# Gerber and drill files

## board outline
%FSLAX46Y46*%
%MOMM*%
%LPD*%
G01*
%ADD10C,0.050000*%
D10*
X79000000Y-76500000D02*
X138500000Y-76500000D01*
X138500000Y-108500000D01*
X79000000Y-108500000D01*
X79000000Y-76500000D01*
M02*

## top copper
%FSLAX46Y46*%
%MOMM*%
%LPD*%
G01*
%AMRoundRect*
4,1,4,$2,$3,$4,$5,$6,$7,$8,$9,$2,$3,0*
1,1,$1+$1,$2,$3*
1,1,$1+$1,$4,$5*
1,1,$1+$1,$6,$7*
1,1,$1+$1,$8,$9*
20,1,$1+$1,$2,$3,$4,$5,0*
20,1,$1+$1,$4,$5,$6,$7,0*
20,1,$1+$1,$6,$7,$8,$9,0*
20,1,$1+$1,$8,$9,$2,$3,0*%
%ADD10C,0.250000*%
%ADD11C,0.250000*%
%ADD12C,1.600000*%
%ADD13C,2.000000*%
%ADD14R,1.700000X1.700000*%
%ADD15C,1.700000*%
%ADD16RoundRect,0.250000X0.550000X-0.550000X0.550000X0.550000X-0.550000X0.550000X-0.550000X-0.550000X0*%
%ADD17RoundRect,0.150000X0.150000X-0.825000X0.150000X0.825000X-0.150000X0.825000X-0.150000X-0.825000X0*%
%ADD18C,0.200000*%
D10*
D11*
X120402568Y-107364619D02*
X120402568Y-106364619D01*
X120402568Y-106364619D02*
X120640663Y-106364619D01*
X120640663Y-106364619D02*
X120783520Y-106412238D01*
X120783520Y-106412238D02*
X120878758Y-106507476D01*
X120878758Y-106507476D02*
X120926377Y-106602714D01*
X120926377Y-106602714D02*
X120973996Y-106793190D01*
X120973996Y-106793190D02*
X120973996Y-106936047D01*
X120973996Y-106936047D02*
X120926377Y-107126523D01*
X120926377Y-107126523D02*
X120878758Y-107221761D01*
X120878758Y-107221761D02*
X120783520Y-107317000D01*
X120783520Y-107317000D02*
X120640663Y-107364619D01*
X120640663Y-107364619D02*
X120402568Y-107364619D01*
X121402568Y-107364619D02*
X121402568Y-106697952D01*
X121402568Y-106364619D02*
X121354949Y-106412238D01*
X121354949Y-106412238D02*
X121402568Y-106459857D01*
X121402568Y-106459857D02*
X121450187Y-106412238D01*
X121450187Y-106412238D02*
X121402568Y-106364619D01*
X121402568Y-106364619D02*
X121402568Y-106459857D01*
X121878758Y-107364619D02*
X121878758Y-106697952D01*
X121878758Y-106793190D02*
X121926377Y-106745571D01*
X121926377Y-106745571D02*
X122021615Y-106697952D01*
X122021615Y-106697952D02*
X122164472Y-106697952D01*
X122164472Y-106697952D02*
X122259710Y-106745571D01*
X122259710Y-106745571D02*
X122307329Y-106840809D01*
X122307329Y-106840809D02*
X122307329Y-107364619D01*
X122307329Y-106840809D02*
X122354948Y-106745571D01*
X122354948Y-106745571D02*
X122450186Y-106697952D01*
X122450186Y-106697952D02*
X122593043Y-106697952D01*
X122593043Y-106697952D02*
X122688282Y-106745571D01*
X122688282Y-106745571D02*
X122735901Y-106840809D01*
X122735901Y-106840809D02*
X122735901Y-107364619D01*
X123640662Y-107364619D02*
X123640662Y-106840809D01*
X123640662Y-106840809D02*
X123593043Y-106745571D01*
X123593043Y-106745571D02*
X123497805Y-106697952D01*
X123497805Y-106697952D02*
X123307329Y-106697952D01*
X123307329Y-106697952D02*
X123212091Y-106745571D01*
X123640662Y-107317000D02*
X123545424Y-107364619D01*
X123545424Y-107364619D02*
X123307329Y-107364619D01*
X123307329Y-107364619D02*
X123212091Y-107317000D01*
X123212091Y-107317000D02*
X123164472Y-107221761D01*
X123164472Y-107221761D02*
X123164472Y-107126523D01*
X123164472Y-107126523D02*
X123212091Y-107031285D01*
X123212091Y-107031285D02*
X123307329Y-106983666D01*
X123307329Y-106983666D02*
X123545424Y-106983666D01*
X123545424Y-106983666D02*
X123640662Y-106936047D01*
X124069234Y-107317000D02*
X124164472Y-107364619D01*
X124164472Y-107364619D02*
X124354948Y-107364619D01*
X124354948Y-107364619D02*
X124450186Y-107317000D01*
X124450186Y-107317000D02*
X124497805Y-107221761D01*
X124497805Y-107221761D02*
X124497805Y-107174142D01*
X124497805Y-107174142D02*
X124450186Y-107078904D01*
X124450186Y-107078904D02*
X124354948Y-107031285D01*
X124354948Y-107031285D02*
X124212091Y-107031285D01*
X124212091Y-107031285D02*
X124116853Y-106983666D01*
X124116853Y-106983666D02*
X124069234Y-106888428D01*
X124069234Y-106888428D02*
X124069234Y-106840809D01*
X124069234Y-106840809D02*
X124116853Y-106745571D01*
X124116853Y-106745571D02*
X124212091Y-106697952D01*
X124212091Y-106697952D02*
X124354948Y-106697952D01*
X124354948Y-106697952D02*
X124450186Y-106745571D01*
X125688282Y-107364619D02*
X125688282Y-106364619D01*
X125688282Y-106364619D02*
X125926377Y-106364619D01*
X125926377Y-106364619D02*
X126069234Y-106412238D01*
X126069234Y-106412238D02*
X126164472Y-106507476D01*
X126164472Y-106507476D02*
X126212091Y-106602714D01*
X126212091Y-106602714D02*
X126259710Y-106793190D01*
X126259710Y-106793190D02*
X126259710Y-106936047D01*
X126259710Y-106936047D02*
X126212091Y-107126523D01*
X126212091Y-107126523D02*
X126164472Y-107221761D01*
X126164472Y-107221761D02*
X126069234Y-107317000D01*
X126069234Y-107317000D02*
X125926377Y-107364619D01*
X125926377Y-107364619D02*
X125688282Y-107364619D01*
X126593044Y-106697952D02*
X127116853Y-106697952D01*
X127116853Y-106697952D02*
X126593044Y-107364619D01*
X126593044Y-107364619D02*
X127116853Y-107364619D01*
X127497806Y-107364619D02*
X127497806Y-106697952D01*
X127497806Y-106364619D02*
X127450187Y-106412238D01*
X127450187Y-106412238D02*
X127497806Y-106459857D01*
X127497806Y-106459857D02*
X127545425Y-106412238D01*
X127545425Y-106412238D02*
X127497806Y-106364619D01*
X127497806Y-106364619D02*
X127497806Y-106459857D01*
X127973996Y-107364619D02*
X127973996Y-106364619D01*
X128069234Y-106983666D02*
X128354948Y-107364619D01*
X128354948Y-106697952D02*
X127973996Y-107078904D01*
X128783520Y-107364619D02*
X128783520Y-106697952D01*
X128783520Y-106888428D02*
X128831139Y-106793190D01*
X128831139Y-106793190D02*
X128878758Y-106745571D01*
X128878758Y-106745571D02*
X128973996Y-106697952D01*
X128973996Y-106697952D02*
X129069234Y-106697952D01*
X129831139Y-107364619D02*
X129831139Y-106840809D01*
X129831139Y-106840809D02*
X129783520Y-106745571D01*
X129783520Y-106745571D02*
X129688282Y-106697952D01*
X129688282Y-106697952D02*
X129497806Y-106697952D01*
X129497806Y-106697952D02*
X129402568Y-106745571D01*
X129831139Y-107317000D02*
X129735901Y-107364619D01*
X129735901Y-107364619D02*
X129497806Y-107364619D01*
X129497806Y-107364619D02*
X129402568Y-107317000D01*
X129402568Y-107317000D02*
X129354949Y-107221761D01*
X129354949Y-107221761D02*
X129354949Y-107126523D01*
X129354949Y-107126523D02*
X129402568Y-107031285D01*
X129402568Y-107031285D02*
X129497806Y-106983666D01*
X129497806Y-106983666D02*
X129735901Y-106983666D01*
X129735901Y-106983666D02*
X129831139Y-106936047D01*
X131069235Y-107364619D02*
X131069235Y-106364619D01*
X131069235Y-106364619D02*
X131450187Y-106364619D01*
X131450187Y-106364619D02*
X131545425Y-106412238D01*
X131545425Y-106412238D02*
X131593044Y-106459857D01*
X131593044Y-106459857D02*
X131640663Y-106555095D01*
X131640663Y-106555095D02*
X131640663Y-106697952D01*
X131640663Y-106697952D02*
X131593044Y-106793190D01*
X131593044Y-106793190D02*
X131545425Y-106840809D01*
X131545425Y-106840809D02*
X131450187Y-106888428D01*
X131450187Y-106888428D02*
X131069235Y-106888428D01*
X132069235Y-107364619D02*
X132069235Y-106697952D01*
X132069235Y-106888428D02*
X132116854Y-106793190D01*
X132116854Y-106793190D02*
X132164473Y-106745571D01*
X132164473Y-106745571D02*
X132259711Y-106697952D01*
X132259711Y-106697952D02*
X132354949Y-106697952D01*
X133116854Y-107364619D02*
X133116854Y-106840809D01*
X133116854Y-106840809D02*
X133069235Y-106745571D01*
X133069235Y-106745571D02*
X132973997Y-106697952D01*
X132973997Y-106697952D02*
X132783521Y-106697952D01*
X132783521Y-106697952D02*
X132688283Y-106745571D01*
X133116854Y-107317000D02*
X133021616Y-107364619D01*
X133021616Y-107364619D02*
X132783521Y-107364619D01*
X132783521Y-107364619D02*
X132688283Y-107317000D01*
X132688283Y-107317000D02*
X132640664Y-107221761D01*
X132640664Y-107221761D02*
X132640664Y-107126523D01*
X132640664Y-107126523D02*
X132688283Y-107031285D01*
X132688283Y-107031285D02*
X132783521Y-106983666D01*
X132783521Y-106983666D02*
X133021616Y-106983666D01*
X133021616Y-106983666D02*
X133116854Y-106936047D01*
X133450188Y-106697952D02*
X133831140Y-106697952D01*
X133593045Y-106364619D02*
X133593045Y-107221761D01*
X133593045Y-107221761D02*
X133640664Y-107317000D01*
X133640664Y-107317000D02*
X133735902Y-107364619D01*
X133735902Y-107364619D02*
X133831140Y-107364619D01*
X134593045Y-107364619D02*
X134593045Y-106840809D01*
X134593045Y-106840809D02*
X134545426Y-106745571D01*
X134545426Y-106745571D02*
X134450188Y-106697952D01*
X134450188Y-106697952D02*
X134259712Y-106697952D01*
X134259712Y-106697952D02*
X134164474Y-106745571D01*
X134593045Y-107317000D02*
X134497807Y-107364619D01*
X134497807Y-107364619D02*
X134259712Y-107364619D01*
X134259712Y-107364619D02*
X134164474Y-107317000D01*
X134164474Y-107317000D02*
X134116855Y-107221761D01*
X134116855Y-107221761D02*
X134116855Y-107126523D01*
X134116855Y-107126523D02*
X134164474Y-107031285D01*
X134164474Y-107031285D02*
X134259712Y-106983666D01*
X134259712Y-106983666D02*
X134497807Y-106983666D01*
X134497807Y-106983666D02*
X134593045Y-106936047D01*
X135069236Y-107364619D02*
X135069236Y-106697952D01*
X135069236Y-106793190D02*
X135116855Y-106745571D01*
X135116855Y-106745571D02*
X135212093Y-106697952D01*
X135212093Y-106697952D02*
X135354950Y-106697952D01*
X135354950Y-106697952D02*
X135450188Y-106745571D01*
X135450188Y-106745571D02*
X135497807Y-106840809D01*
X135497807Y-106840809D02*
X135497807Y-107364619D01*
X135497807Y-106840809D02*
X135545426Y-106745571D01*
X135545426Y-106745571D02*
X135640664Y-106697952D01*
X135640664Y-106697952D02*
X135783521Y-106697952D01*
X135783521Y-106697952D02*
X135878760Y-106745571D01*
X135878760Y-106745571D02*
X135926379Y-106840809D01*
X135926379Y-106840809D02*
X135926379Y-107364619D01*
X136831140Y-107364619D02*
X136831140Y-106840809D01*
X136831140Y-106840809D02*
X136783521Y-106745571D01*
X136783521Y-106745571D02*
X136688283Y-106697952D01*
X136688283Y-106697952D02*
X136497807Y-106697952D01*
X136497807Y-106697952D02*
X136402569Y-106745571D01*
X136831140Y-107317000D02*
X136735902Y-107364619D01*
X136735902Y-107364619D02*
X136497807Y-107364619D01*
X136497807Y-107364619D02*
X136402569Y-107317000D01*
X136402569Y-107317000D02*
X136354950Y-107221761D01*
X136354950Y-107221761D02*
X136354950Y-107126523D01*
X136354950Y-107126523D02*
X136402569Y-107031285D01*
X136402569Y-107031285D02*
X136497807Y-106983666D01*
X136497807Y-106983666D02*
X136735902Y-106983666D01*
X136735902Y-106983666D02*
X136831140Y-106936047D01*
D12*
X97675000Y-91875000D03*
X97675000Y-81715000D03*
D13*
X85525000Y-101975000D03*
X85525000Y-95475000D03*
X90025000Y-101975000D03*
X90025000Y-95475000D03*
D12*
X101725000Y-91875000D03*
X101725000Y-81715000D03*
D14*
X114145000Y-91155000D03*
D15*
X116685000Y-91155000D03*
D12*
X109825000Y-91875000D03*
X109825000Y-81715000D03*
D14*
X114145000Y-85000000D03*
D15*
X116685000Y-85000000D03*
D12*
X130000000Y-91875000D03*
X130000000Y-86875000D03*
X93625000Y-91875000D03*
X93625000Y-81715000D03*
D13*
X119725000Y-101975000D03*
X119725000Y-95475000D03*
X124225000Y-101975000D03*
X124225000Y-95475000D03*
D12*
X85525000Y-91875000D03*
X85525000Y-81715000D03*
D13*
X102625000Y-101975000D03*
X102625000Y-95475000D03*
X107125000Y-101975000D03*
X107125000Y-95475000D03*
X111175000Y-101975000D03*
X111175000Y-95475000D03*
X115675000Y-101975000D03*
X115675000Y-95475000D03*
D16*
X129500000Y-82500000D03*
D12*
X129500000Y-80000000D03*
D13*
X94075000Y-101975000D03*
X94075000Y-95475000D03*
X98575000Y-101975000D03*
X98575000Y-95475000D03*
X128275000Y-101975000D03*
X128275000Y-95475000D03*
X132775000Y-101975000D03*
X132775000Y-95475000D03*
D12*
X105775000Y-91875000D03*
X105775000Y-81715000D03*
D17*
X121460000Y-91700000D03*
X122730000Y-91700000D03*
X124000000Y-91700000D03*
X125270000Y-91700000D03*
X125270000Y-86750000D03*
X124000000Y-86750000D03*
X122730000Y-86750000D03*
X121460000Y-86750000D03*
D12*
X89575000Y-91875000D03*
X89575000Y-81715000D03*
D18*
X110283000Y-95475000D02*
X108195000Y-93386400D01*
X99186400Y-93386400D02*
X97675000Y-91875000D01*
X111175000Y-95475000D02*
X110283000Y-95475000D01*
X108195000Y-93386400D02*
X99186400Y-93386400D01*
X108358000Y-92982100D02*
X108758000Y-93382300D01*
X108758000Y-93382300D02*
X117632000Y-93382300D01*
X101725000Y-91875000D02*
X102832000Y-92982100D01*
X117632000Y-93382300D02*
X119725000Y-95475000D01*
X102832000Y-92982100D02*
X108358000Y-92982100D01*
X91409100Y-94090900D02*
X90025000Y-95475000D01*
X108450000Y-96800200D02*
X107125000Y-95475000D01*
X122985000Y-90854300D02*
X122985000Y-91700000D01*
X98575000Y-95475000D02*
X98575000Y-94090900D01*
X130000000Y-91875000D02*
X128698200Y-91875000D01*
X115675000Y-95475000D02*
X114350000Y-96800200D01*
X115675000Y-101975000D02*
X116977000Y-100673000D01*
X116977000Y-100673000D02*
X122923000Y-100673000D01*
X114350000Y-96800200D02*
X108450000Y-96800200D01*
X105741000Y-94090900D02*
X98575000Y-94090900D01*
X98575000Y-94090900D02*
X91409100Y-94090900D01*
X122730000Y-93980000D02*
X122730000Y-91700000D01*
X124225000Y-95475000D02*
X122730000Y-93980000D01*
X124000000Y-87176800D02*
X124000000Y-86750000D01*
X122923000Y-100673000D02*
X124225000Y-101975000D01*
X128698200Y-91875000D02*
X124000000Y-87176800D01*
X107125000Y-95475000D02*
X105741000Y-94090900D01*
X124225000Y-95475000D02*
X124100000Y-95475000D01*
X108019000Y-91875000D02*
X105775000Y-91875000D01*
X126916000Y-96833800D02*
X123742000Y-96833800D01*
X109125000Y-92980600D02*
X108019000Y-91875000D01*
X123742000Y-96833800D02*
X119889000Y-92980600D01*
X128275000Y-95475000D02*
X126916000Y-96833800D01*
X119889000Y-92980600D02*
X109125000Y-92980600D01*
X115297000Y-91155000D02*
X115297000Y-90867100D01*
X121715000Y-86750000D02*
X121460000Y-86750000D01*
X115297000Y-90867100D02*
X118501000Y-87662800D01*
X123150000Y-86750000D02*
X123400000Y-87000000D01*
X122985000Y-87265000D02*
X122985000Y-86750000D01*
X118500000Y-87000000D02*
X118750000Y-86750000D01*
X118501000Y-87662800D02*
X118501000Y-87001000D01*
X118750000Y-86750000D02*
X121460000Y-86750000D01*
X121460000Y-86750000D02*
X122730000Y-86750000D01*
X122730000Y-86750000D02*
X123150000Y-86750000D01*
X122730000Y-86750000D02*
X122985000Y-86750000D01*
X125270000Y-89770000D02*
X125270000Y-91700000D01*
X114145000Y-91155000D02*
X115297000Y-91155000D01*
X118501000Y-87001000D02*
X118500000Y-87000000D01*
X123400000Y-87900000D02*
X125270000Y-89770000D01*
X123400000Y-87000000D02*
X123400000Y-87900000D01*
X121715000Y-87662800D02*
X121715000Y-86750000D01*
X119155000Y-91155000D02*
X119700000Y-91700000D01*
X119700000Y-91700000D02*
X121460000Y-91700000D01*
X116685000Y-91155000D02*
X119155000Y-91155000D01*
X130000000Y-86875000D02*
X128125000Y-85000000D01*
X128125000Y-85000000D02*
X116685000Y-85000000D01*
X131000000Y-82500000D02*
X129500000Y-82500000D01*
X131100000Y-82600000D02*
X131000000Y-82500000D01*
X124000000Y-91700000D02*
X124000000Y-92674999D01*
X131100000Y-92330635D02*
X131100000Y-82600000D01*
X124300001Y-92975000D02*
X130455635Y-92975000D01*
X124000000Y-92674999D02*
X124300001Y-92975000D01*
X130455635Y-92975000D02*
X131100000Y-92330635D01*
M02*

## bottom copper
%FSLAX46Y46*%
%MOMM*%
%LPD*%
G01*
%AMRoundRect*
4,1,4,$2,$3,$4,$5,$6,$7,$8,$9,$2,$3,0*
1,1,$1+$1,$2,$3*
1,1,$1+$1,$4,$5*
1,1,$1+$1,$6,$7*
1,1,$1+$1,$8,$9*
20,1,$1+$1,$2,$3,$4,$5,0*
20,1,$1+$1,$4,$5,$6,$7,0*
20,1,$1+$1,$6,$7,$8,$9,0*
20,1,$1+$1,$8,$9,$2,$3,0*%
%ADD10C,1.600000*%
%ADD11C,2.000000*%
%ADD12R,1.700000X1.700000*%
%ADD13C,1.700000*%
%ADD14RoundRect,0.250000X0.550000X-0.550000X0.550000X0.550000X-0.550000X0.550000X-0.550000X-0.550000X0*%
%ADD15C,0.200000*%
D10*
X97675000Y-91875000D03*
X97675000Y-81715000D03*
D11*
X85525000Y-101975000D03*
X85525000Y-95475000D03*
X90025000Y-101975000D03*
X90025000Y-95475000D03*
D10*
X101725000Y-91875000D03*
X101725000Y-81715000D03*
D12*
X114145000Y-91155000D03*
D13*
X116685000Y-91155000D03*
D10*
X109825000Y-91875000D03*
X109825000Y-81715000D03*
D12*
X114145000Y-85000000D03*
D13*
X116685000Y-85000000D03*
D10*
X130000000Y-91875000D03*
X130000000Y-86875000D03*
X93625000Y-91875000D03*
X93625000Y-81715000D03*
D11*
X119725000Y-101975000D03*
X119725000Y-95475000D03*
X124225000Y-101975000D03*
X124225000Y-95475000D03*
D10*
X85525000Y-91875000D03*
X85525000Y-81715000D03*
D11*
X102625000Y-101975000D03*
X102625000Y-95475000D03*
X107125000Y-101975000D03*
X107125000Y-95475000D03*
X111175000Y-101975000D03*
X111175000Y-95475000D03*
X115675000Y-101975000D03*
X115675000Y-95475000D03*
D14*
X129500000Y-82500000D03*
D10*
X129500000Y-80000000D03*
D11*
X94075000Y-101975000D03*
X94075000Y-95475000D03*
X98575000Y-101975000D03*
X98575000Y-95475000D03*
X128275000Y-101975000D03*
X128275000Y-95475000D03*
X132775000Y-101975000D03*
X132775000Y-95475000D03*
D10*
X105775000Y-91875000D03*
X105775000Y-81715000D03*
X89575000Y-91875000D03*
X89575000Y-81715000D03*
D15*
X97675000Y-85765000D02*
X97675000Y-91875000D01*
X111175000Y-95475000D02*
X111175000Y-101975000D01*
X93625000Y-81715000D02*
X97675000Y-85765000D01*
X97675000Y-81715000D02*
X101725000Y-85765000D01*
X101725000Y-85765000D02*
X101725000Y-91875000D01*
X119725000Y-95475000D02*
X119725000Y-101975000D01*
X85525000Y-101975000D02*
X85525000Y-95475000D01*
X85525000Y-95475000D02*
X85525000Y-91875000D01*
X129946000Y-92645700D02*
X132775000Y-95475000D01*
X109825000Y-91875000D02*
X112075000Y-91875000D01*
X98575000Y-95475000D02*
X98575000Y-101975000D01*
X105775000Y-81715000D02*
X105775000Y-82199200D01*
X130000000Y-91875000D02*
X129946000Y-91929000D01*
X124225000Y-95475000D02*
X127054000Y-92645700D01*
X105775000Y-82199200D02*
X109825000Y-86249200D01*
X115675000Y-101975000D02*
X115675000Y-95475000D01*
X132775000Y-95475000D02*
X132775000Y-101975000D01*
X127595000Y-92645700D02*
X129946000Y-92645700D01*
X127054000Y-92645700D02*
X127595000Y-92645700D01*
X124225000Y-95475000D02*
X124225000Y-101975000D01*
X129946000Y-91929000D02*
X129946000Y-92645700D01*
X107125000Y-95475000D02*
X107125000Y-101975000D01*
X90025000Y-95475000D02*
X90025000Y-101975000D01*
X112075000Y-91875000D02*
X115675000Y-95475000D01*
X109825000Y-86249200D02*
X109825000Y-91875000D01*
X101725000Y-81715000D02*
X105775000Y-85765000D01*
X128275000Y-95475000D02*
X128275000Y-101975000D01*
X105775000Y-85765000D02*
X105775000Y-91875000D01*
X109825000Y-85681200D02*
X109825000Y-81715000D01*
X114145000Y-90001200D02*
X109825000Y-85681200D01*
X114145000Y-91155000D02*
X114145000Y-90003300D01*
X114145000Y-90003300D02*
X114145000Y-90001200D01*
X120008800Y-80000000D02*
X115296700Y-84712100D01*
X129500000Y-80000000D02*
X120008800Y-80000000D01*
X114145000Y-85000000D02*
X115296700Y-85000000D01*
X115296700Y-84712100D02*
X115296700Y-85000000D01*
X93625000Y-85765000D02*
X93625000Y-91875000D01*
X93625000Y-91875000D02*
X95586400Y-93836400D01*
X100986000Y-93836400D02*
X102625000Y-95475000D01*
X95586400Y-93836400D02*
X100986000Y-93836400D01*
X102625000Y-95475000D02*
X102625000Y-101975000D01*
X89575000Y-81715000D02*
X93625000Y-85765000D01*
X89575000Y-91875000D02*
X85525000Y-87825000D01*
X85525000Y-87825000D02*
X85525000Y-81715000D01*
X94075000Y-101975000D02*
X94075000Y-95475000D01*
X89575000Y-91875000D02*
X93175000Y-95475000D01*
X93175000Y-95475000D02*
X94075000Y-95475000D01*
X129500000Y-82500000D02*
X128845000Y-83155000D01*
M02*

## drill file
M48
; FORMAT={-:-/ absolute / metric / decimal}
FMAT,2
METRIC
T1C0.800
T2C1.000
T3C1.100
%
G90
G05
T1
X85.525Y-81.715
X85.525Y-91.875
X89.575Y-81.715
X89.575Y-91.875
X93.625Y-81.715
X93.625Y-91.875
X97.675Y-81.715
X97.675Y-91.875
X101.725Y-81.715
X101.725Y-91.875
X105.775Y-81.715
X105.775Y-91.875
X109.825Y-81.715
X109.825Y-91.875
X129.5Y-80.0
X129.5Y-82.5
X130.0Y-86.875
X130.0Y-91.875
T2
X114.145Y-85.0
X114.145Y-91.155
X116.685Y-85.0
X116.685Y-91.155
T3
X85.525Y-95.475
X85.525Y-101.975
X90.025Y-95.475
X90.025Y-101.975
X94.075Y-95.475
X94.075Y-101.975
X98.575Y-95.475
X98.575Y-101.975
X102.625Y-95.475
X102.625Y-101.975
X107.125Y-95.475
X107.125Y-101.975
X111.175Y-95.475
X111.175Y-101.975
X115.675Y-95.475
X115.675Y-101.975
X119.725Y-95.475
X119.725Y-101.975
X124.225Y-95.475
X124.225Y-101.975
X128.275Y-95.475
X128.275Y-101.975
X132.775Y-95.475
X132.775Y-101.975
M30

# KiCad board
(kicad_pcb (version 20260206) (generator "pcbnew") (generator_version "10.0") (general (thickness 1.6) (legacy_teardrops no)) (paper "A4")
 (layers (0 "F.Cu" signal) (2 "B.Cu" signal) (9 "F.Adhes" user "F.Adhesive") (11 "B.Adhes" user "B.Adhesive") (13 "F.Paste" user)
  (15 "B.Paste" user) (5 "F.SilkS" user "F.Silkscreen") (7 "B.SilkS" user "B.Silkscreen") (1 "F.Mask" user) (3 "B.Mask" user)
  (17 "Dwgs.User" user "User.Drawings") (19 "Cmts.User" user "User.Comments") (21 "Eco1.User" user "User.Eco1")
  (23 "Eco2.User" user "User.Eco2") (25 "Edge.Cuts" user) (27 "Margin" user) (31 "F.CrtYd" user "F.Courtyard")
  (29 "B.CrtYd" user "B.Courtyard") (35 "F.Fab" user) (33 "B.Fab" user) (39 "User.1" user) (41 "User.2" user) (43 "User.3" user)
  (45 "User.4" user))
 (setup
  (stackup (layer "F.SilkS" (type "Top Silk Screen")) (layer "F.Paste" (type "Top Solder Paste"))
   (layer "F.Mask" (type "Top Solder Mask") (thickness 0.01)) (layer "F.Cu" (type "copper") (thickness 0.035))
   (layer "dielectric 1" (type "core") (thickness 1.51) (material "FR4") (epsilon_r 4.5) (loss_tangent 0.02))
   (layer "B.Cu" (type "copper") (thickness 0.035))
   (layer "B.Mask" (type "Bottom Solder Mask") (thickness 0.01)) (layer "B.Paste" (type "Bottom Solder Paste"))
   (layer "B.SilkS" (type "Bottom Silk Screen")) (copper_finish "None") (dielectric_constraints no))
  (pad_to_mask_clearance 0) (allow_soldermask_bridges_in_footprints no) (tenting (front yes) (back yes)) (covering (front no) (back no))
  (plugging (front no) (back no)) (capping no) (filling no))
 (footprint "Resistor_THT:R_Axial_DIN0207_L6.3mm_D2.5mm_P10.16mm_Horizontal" (layer "F.Cu") (at 97.675 91.875 90)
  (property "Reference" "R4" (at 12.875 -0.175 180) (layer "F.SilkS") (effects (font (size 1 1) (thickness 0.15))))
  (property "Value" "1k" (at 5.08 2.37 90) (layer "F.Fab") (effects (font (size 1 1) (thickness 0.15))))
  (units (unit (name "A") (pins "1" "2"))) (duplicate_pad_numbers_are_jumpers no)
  (pad "1" thru_hole circle (at 0 0 90) (size 1.6 1.6) (drill 0.8) (layers "*.Cu" "*.Mask") (remove_unused_layers no) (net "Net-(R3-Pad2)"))
  (pad "2" thru_hole circle (at 10.16 0 90) (size 1.6 1.6) (drill 0.8) (layers "*.Cu" "*.Mask") (remove_unused_layers no)
   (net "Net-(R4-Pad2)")))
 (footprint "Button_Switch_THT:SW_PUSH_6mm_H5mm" (layer "F.Cu") (at 85.525 101.975 90)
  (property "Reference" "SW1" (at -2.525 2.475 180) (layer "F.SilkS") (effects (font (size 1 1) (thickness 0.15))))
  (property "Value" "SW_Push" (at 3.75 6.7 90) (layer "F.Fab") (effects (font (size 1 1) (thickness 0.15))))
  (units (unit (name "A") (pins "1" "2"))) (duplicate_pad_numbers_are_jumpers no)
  (pad "1" thru_hole circle (at 0 0 180) (size 2 2) (drill 1.1) (layers "*.Cu" "*.Mask") (remove_unused_layers no) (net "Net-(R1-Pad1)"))
  (pad "1" thru_hole circle (at 6.5 0 180) (size 2 2) (drill 1.1) (layers "*.Cu" "*.Mask") (remove_unused_layers no) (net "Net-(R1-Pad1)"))
  (pad "2" thru_hole circle (at 0 4.5 180) (size 2 2) (drill 1.1) (layers "*.Cu" "*.Mask") (remove_unused_layers no) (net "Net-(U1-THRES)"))
  (pad "2" thru_hole circle (at 6.5 4.5 180) (size 2 2) (drill 1.1) (layers "*.Cu" "*.Mask") (remove_unused_layers no)
   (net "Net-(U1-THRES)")))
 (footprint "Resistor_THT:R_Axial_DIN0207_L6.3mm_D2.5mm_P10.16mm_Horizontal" (layer "F.Cu") (at 101.725 91.875 90)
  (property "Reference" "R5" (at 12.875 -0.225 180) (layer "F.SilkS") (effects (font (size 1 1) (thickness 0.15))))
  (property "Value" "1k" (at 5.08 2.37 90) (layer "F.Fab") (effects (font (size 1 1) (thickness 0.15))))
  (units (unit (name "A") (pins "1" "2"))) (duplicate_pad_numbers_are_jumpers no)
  (pad "1" thru_hole circle (at 0 0 90) (size 1.6 1.6) (drill 0.8) (layers "*.Cu" "*.Mask") (remove_unused_layers no) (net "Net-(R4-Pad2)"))
  (pad "2" thru_hole circle (at 10.16 0 90) (size 1.6 1.6) (drill 0.8) (layers "*.Cu" "*.Mask") (remove_unused_layers no)
   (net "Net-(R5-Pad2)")))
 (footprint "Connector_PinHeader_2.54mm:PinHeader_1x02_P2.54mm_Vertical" (layer "F.Cu") (at 114.145 91.155 90)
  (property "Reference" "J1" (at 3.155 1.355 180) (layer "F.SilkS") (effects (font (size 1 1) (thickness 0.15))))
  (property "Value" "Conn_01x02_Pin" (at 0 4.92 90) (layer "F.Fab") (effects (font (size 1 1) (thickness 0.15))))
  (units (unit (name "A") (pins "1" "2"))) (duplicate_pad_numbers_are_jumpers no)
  (pad "1" thru_hole rect (at 0 0 90) (size 1.7 1.7) (drill 1) (layers "*.Cu" "*.Mask") (remove_unused_layers no) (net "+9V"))
  (pad "2" thru_hole circle (at 0 2.54 90) (size 1.7 1.7) (drill 1) (layers "*.Cu" "*.Mask") (remove_unused_layers no) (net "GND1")))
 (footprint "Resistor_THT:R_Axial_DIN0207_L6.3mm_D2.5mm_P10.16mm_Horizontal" (layer "F.Cu") (at 109.825 91.875 90)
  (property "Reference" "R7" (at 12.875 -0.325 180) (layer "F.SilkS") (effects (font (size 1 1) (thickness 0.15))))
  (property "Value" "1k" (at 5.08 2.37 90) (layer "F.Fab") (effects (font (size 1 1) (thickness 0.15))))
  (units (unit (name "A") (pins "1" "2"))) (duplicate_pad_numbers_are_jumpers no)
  (pad "1" thru_hole circle (at 0 0 90) (size 1.6 1.6) (drill 0.8) (layers "*.Cu" "*.Mask") (remove_unused_layers no) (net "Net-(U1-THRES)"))
  (pad "2" thru_hole circle (at 10.16 0 90) (size 1.6 1.6) (drill 0.8) (layers "*.Cu" "*.Mask") (remove_unused_layers no) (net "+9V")))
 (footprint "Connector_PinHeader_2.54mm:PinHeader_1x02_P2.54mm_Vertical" (layer "F.Cu") (at 114.145 85 90)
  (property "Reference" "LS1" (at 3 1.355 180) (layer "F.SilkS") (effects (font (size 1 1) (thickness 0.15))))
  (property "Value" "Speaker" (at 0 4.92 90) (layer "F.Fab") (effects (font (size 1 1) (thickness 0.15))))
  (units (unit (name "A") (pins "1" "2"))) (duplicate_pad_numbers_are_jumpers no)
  (pad "1" thru_hole rect (at 0 0 90) (size 1.7 1.7) (drill 1) (layers "*.Cu" "*.Mask") (remove_unused_layers no) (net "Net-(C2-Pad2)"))
  (pad "2" thru_hole circle (at 0 2.54 90) (size 1.7 1.7) (drill 1) (layers "*.Cu" "*.Mask") (remove_unused_layers no) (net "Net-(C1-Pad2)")))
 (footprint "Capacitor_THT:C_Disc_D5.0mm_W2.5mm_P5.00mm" (layer "F.Cu") (at 130 91.875 90)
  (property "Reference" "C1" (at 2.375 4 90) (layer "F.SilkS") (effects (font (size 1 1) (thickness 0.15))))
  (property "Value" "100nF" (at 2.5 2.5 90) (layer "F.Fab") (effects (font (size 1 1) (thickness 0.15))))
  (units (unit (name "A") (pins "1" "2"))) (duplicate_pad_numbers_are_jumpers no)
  (pad "1" thru_hole circle (at 0 0 90) (size 1.6 1.6) (drill 0.8) (layers "*.Cu" "*.Mask") (remove_unused_layers no) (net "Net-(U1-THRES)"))
  (pad "2" thru_hole circle (at 5 0 90) (size 1.6 1.6) (drill 0.8) (layers "*.Cu" "*.Mask") (remove_unused_layers no) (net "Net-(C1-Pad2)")))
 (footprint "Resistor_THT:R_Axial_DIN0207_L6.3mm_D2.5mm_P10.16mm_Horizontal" (layer "F.Cu") (at 93.625 91.875 90)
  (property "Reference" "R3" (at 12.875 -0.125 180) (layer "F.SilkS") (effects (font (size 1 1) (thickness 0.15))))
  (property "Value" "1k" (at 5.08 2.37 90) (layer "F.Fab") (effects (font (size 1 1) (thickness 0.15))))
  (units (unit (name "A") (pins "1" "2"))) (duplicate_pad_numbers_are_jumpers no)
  (pad "1" thru_hole circle (at 0 0 90) (size 1.6 1.6) (drill 0.8) (layers "*.Cu" "*.Mask") (remove_unused_layers no) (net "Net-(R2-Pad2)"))
  (pad "2" thru_hole circle (at 10.16 0 90) (size 1.6 1.6) (drill 0.8) (layers "*.Cu" "*.Mask") (remove_unused_layers no)
   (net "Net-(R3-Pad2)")))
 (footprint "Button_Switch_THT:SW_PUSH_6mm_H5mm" (layer "F.Cu") (at 119.725 101.975 90)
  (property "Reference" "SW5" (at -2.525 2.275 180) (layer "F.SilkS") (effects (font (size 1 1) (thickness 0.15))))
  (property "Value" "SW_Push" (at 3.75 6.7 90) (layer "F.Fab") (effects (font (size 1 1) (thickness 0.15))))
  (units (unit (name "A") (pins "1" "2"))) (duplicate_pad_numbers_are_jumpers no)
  (pad "1" thru_hole circle (at 0 0 180) (size 2 2) (drill 1.1) (layers "*.Cu" "*.Mask") (remove_unused_layers no) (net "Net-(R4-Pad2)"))
  (pad "1" thru_hole circle (at 6.5 0 180) (size 2 2) (drill 1.1) (layers "*.Cu" "*.Mask") (remove_unused_layers no) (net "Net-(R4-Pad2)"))
  (pad "2" thru_hole circle (at 0 4.5 180) (size 2 2) (drill 1.1) (layers "*.Cu" "*.Mask") (remove_unused_layers no) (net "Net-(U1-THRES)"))
  (pad "2" thru_hole circle (at 6.5 4.5 180) (size 2 2) (drill 1.1) (layers "*.Cu" "*.Mask") (remove_unused_layers no)
   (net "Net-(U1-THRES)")))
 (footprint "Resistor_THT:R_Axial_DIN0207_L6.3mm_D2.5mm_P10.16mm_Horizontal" (layer "F.Cu") (at 85.525 91.875 90)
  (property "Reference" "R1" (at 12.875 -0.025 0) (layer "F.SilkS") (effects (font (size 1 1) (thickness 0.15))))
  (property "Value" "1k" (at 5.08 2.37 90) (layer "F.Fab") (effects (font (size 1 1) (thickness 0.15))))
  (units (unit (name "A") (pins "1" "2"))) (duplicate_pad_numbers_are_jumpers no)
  (pad "1" thru_hole circle (at 0 0 90) (size 1.6 1.6) (drill 0.8) (layers "*.Cu" "*.Mask") (remove_unused_layers no) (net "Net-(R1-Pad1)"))
  (pad "2" thru_hole circle (at 10.16 0 90) (size 1.6 1.6) (drill 0.8) (layers "*.Cu" "*.Mask") (remove_unused_layers no)
   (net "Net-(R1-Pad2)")))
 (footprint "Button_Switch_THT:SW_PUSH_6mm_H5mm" (layer "F.Cu") (at 102.625 101.975 90)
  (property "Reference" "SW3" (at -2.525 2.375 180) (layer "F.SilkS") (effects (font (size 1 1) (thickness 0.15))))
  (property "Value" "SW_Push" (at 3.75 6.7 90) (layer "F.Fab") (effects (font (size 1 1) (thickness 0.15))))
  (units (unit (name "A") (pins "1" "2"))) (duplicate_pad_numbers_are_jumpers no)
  (pad "1" thru_hole circle (at 0 0 180) (size 2 2) (drill 1.1) (layers "*.Cu" "*.Mask") (remove_unused_layers no) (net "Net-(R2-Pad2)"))
  (pad "1" thru_hole circle (at 6.5 0 180) (size 2 2) (drill 1.1) (layers "*.Cu" "*.Mask") (remove_unused_layers no) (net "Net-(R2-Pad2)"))
  (pad "2" thru_hole circle (at 0 4.5 180) (size 2 2) (drill 1.1) (layers "*.Cu" "*.Mask") (remove_unused_layers no) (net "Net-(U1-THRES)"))
  (pad "2" thru_hole circle (at 6.5 4.5 180) (size 2 2) (drill 1.1) (layers "*.Cu" "*.Mask") (remove_unused_layers no)
   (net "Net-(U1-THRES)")))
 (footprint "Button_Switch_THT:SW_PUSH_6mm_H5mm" (layer "F.Cu") (at 111.175 101.975 90)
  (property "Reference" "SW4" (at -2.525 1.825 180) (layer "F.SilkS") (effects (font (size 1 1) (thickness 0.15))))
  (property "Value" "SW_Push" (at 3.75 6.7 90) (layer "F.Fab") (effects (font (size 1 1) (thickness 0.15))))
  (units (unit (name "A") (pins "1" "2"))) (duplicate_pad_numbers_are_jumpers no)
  (pad "1" thru_hole circle (at 0 0 180) (size 2 2) (drill 1.1) (layers "*.Cu" "*.Mask") (remove_unused_layers no) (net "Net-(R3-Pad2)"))
  (pad "1" thru_hole circle (at 6.5 0 180) (size 2 2) (drill 1.1) (layers "*.Cu" "*.Mask") (remove_unused_layers no) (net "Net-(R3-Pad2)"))
  (pad "2" thru_hole circle (at 0 4.5 180) (size 2 2) (drill 1.1) (layers "*.Cu" "*.Mask") (remove_unused_layers no) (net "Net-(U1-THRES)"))
  (pad "2" thru_hole circle (at 6.5 4.5 180) (size 2 2) (drill 1.1) (layers "*.Cu" "*.Mask") (remove_unused_layers no)
   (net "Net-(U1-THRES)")))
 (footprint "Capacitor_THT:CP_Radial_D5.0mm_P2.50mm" (layer "F.Cu") (at 129.5 82.5 90)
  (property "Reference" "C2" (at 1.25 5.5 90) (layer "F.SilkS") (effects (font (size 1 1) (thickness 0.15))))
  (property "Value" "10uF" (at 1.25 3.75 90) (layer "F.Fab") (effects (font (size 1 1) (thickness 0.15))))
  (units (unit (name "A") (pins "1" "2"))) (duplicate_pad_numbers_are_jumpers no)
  (pad "1" thru_hole roundrect (at 0 0 90) (size 1.6 1.6) (drill 0.8) (layers "*.Cu" "*.Mask") (remove_unused_layers no)
   (roundrect_rratio 0.15625) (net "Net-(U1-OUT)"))
  (pad "2" thru_hole circle (at 2.5 0 90) (size 1.6 1.6) (drill 0.8) (layers "*.Cu" "*.Mask") (remove_unused_layers no)
   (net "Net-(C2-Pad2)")))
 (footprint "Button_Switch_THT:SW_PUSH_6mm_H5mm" (layer "F.Cu") (at 94.075 101.975 90)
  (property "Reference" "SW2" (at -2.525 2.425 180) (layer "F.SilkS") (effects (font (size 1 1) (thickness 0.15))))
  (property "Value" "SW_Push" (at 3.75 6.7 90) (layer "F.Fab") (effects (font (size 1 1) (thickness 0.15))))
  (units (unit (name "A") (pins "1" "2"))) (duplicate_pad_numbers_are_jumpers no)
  (pad "1" thru_hole circle (at 0 0 180) (size 2 2) (drill 1.1) (layers "*.Cu" "*.Mask") (remove_unused_layers no) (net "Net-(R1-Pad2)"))
  (pad "1" thru_hole circle (at 6.5 0 180) (size 2 2) (drill 1.1) (layers "*.Cu" "*.Mask") (remove_unused_layers no) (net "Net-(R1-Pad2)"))
  (pad "2" thru_hole circle (at 0 4.5 180) (size 2 2) (drill 1.1) (layers "*.Cu" "*.Mask") (remove_unused_layers no) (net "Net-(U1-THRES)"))
  (pad "2" thru_hole circle (at 6.5 4.5 180) (size 2 2) (drill 1.1) (layers "*.Cu" "*.Mask") (remove_unused_layers no)
   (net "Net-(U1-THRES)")))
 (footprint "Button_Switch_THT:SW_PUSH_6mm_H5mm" (layer "F.Cu") (at 128.275 101.975 90)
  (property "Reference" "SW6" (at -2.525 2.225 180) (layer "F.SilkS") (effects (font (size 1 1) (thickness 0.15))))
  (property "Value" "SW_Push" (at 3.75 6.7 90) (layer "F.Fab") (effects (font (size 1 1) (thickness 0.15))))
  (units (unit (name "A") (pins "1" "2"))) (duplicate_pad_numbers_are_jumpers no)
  (pad "1" thru_hole circle (at 0 0 180) (size 2 2) (drill 1.1) (layers "*.Cu" "*.Mask") (remove_unused_layers no) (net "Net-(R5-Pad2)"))
  (pad "1" thru_hole circle (at 6.5 0 180) (size 2 2) (drill 1.1) (layers "*.Cu" "*.Mask") (remove_unused_layers no) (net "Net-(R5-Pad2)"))
  (pad "2" thru_hole circle (at 0 4.5 180) (size 2 2) (drill 1.1) (layers "*.Cu" "*.Mask") (remove_unused_layers no) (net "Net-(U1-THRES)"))
  (pad "2" thru_hole circle (at 6.5 4.5 180) (size 2 2) (drill 1.1) (layers "*.Cu" "*.Mask") (remove_unused_layers no)
   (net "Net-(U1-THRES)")))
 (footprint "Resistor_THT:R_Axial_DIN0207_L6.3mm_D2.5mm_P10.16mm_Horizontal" (layer "F.Cu") (at 105.775 91.875 90)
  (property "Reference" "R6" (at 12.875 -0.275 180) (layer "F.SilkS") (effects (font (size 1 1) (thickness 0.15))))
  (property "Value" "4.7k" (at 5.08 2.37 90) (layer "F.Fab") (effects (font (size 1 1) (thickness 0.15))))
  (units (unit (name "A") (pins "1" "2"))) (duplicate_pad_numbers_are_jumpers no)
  (pad "1" thru_hole circle (at 0 0 90) (size 1.6 1.6) (drill 0.8) (layers "*.Cu" "*.Mask") (remove_unused_layers no) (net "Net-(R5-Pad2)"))
  (pad "2" thru_hole circle (at 10.16 0 90) (size 1.6 1.6) (drill 0.8) (layers "*.Cu" "*.Mask") (remove_unused_layers no)
   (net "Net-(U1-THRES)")))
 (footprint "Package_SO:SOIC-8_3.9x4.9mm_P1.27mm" (layer "F.Cu") (at 123.365 89.225 90)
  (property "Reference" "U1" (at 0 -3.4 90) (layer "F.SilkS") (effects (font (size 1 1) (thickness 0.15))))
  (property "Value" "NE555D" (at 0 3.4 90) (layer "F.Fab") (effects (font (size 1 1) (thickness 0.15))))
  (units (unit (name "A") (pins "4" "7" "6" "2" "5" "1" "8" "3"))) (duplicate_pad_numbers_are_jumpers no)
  (pad "1" smd roundrect (at -2.475 -1.905 90) (size 1.95 0.6) (layers "F.Cu" "F.Mask" "F.Paste") (roundrect_rratio 0.25) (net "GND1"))
  (pad "2" smd roundrect (at -2.475 -0.635 90) (size 1.95 0.6) (layers "F.Cu" "F.Mask" "F.Paste") (roundrect_rratio 0.25)
   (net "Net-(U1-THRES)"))
  (pad "3" smd roundrect (at -2.475 0.635 90) (size 1.95 0.6) (layers "F.Cu" "F.Mask" "F.Paste") (roundrect_rratio 0.25)
   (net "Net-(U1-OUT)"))
  (pad "4" smd roundrect (at -2.475 1.905 90) (size 1.95 0.6) (layers "F.Cu" "F.Mask" "F.Paste") (roundrect_rratio 0.25) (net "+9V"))
  (pad "5" smd roundrect (at 2.475 1.905 90) (size 1.95 0.6) (layers "F.Cu" "F.Mask" "F.Paste") (roundrect_rratio 0.25)
   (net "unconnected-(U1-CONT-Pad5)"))
  (pad "6" smd roundrect (at 2.475 0.635 90) (size 1.95 0.6) (layers "F.Cu" "F.Mask" "F.Paste") (roundrect_rratio 0.25)
   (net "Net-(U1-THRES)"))
  (pad "7" smd roundrect (at 2.475 -0.635 90) (size 1.95 0.6) (layers "F.Cu" "F.Mask" "F.Paste") (roundrect_rratio 0.25) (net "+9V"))
  (pad "8" smd roundrect (at 2.475 -1.905 90) (size 1.95 0.6) (layers "F.Cu" "F.Mask" "F.Paste") (roundrect_rratio 0.25) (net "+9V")))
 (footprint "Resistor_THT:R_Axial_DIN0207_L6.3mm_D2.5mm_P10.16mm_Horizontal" (layer "F.Cu") (at 89.575 91.875 90)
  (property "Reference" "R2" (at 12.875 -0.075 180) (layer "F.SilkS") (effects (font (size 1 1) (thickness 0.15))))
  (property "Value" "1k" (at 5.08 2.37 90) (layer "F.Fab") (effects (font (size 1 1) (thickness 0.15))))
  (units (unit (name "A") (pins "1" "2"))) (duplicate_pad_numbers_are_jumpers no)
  (pad "1" thru_hole circle (at 0 0 90) (size 1.6 1.6) (drill 0.8) (layers "*.Cu" "*.Mask") (remove_unused_layers no) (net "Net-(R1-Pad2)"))
  (pad "2" thru_hole circle (at 10.16 0 90) (size 1.6 1.6) (drill 0.8) (layers "*.Cu" "*.Mask") (remove_unused_layers no)
   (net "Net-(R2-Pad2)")))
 (gr_rect (start 79 76.5) (end 138.5 108.5) (stroke (width 0.05) (type default)) (fill no) (layer "Edge.Cuts"))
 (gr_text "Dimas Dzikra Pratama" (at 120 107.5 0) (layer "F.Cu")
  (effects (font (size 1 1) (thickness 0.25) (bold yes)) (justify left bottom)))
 (segment (start 110.283 95.475) (end 108.195 93.3864) (width 0.2) (layer "F.Cu") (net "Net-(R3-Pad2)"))
 (segment (start 99.1864 93.3864) (end 97.675 91.875) (width 0.2) (layer "F.Cu") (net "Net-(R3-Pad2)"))
 (segment (start 111.175 95.475) (end 110.283 95.475) (width 0.2) (layer "F.Cu") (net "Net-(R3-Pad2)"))
 (segment (start 108.195 93.3864) (end 99.1864 93.3864) (width 0.2) (layer "F.Cu") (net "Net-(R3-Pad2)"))
 (segment (start 97.675 85.765) (end 97.675 91.875) (width 0.2) (layer "B.Cu") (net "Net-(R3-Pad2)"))
 (segment (start 111.175 95.475) (end 111.175 101.975) (width 0.2) (layer "B.Cu") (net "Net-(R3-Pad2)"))
 (segment (start 93.625 81.715) (end 97.675 85.765) (width 0.2) (layer "B.Cu") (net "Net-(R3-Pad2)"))
 (segment (start 108.358 92.9821) (end 108.758 93.3823) (width 0.2) (layer "F.Cu") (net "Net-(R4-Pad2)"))
 (segment (start 108.758 93.3823) (end 117.632 93.3823) (width 0.2) (layer "F.Cu") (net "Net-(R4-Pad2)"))
 (segment (start 101.725 91.875) (end 102.832 92.9821) (width 0.2) (layer "F.Cu") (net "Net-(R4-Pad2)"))
 (segment (start 117.632 93.3823) (end 119.725 95.475) (width 0.2) (layer "F.Cu") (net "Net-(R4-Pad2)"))
 (segment (start 102.832 92.9821) (end 108.358 92.9821) (width 0.2) (layer "F.Cu") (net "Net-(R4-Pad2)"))
 (segment (start 97.675 81.715) (end 101.725 85.765) (width 0.2) (layer "B.Cu") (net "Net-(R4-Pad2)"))
 (segment (start 101.725 85.765) (end 101.725 91.875) (width 0.2) (layer "B.Cu") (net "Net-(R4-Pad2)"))
 (segment (start 119.725 95.475) (end 119.725 101.975) (width 0.2) (layer "B.Cu") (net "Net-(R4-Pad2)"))
 (segment (start 85.525 101.975) (end 85.525 95.475) (width 0.2) (layer "B.Cu") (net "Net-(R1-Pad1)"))
 (segment (start 85.525 95.475) (end 85.525 91.875) (width 0.2) (layer "B.Cu") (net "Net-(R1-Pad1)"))
 (segment (start 91.4091 94.0909) (end 90.025 95.475) (width 0.2) (layer "F.Cu") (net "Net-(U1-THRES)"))
 (segment (start 108.45 96.8002) (end 107.125 95.475) (width 0.2) (layer "F.Cu") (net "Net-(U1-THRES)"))
 (segment (start 122.985 90.8543) (end 122.985 91.7) (width 0.2) (layer "F.Cu") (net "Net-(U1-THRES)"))
 (segment (start 98.575 95.475) (end 98.575 94.0909) (width 0.2) (layer "F.Cu") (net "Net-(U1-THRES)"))
 (segment (start 130 91.875) (end 128.6982 91.875) (width 0.2) (layer "F.Cu") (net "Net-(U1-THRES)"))
 (segment (start 115.675 95.475) (end 114.35 96.8002) (width 0.2) (layer "F.Cu") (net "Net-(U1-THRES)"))
 (segment (start 115.675 101.975) (end 116.977 100.673) (width 0.2) (layer "F.Cu") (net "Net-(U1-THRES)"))
 (segment (start 116.977 100.673) (end 122.923 100.673) (width 0.2) (layer "F.Cu") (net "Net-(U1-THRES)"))
 (segment (start 114.35 96.8002) (end 108.45 96.8002) (width 0.2) (layer "F.Cu") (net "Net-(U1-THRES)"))
 (segment (start 105.741 94.0909) (end 98.575 94.0909) (width 0.2) (layer "F.Cu") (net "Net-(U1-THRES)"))
 (segment (start 98.575 94.0909) (end 91.4091 94.0909) (width 0.2) (layer "F.Cu") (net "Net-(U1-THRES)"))
 (segment (start 122.73 93.98) (end 122.73 91.7) (width 0.2) (layer "F.Cu") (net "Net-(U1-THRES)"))
 (segment (start 124.225 95.475) (end 122.73 93.98) (width 0.2) (layer "F.Cu") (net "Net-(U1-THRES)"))
 (segment (start 124 87.1768) (end 124 86.75) (width 0.2) (layer "F.Cu") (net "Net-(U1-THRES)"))
 (segment (start 122.923 100.673) (end 124.225 101.975) (width 0.2) (layer "F.Cu") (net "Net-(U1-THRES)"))
 (segment (start 128.6982 91.875) (end 124 87.1768) (width 0.2) (layer "F.Cu") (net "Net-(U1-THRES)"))
 (segment (start 107.125 95.475) (end 105.741 94.0909) (width 0.2) (layer "F.Cu") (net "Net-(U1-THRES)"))
 (segment (start 124.225 95.475) (end 124.1 95.475) (width 0.2) (layer "F.Cu") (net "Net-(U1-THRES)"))
 (segment (start 129.946 92.6457) (end 132.775 95.475) (width 0.2) (layer "B.Cu") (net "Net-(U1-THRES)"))
 (segment (start 109.825 91.875) (end 112.075 91.875) (width 0.2) (layer "B.Cu") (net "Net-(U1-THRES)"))
 (segment (start 98.575 95.475) (end 98.575 101.975) (width 0.2) (layer "B.Cu") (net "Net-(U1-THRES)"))
 (segment (start 105.775 81.715) (end 105.775 82.1992) (width 0.2) (layer "B.Cu") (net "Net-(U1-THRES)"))
 (segment (start 130 91.875) (end 129.946 91.929) (width 0.2) (layer "B.Cu") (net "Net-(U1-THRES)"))
 (segment (start 124.225 95.475) (end 127.054 92.6457) (width 0.2) (layer "B.Cu") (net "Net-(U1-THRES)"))
 (segment (start 105.775 82.1992) (end 109.825 86.2492) (width 0.2) (layer "B.Cu") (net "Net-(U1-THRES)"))
 (segment (start 115.675 101.975) (end 115.675 95.475) (width 0.2) (layer "B.Cu") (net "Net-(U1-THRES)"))
 (segment (start 132.775 95.475) (end 132.775 101.975) (width 0.2) (layer "B.Cu") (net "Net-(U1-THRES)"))
 (segment (start 127.595 92.6457) (end 129.946 92.6457) (width 0.2) (layer "B.Cu") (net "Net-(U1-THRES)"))
 (segment (start 127.054 92.6457) (end 127.595 92.6457) (width 0.2) (layer "B.Cu") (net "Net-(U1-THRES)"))
 (segment (start 124.225 95.475) (end 124.225 101.975) (width 0.2) (layer "B.Cu") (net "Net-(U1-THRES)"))
 (segment (start 129.946 91.929) (end 129.946 92.6457) (width 0.2) (layer "B.Cu") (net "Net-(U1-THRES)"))
 (segment (start 107.125 95.475) (end 107.125 101.975) (width 0.2) (layer "B.Cu") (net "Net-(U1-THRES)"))
 (segment (start 90.025 95.475) (end 90.025 101.975) (width 0.2) (layer "B.Cu") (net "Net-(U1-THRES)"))
 (segment (start 112.075 91.875) (end 115.675 95.475) (width 0.2) (layer "B.Cu") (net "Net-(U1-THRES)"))
 (segment (start 109.825 86.2492) (end 109.825 91.875) (width 0.2) (layer "B.Cu") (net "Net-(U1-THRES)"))
 (segment (start 108.019 91.875) (end 105.775 91.875) (width 0.2) (layer "F.Cu") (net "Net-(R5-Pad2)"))
 (segment (start 126.916 96.8338) (end 123.742 96.8338) (width 0.2) (layer "F.Cu") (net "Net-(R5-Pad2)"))
 (segment (start 109.125 92.9806) (end 108.019 91.875) (width 0.2) (layer "F.Cu") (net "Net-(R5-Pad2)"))
 (segment (start 123.742 96.8338) (end 119.889 92.9806) (width 0.2) (layer "F.Cu") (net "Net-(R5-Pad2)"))
 (segment (start 128.275 95.475) (end 126.916 96.8338) (width 0.2) (layer "F.Cu") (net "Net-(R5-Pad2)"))
 (segment (start 119.889 92.9806) (end 109.125 92.9806) (width 0.2) (layer "F.Cu") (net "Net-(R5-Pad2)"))
 (segment (start 101.725 81.715) (end 105.775 85.765) (width 0.2) (layer "B.Cu") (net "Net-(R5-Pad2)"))
 (segment (start 128.275 95.475) (end 128.275 101.975) (width 0.2) (layer "B.Cu") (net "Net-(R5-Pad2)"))
 (segment (start 105.775 85.765) (end 105.775 91.875) (width 0.2) (layer "B.Cu") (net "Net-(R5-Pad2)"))
 (segment (start 115.297 91.155) (end 115.297 90.8671) (width 0.2) (layer "F.Cu") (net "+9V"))
 (segment (start 121.715 86.75) (end 121.46 86.75) (width 0.2) (layer "F.Cu") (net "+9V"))
 (segment (start 115.297 90.8671) (end 118.501 87.6628) (width 0.2) (layer "F.Cu") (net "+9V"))
 (segment (start 123.15 86.75) (end 123.4 87) (width 0.2) (layer "F.Cu") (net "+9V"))
 (segment (start 122.985 87.265) (end 122.985 86.75) (width 0.2) (layer "F.Cu") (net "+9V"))
 (segment (start 118.5 87) (end 118.75 86.75) (width 0.2) (layer "F.Cu") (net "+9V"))
 (segment (start 118.501 87.6628) (end 118.501 87.001) (width 0.2) (layer "F.Cu") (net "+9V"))
 (segment (start 118.75 86.75) (end 121.46 86.75) (width 0.2) (layer "F.Cu") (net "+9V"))
 (segment (start 121.46 86.75) (end 122.73 86.75) (width 0.2) (layer "F.Cu") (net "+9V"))
 (segment (start 122.73 86.75) (end 123.15 86.75) (width 0.2) (layer "F.Cu") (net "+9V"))
 (segment (start 122.73 86.75) (end 122.985 86.75) (width 0.2) (layer "F.Cu") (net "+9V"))
 (segment (start 125.27 89.77) (end 125.27 91.7) (width 0.2) (layer "F.Cu") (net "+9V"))
 (segment (start 114.145 91.155) (end 115.297 91.155) (width 0.2) (layer "F.Cu") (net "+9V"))
 (segment (start 118.501 87.001) (end 118.5 87) (width 0.2) (layer "F.Cu") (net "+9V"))
 (segment (start 123.4 87.9) (end 125.27 89.77) (width 0.2) (layer "F.Cu") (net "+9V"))
 (segment (start 123.4 87) (end 123.4 87.9) (width 0.2) (layer "F.Cu") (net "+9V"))
 (segment (start 121.715 87.6628) (end 121.715 86.75) (width 0.2) (layer "F.Cu") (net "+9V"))
 (segment (start 109.825 85.6812) (end 109.825 81.715) (width 0.2) (layer "B.Cu") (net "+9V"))
 (segment (start 114.145 90.0012) (end 109.825 85.6812) (width 0.2) (layer "B.Cu") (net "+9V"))
 (segment (start 114.145 91.155) (end 114.145 90.0033) (width 0.2) (layer "B.Cu") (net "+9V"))
 (segment (start 114.145 90.0033) (end 114.145 90.0012) (width 0.2) (layer "B.Cu") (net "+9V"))
 (segment (start 119.155 91.155) (end 119.7 91.7) (width 0.2) (layer "F.Cu") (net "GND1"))
 (segment (start 119.7 91.7) (end 121.46 91.7) (width 0.2) (layer "F.Cu") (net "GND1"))
 (segment (start 116.685 91.155) (end 119.155 91.155) (width 0.2) (layer "F.Cu") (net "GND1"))
 (segment (start 120.0088 80) (end 115.2967 84.7121) (width 0.2) (layer "B.Cu") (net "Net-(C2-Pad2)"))
 (segment (start 129.5 80) (end 120.0088 80) (width 0.2) (layer "B.Cu") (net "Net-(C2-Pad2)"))
 (segment (start 114.145 85) (end 115.2967 85) (width 0.2) (layer "B.Cu") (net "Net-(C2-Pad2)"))
 (segment (start 115.2967 84.7121) (end 115.2967 85) (width 0.2) (layer "B.Cu") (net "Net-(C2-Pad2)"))
 (segment (start 130 86.875) (end 128.125 85) (width 0.2) (layer "F.Cu") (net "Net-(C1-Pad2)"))
 (segment (start 128.125 85) (end 116.685 85) (width 0.2) (layer "F.Cu") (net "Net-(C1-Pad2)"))
 (segment (start 93.625 85.765) (end 93.625 91.875) (width 0.2) (layer "B.Cu") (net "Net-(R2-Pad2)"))
 (segment (start 93.625 91.875) (end 95.5864 93.8364) (width 0.2) (layer "B.Cu") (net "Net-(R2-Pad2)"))
 (segment (start 100.986 93.8364) (end 102.625 95.475) (width 0.2) (layer "B.Cu") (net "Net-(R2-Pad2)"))
 (segment (start 95.5864 93.8364) (end 100.986 93.8364) (width 0.2) (layer "B.Cu") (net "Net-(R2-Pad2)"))
 (segment (start 102.625 95.475) (end 102.625 101.975) (width 0.2) (layer "B.Cu") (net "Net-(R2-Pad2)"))
 (segment (start 89.575 81.715) (end 93.625 85.765) (width 0.2) (layer "B.Cu") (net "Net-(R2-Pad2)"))
 (segment (start 89.575 91.875) (end 85.525 87.825) (width 0.2) (layer "B.Cu") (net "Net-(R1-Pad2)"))
 (segment (start 85.525 87.825) (end 85.525 81.715) (width 0.2) (layer "B.Cu") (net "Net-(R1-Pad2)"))
 (segment (start 94.075 101.975) (end 94.075 95.475) (width 0.2) (layer "B.Cu") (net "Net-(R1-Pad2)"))
 (segment (start 89.575 91.875) (end 93.175 95.475) (width 0.2) (layer "B.Cu") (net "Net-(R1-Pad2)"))
 (segment (start 93.175 95.475) (end 94.075 95.475) (width 0.2) (layer "B.Cu") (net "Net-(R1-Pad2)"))
 (segment (start 131 82.5) (end 129.5 82.5) (width 0.2) (layer "F.Cu") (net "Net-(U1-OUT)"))
 (segment (start 131.1 82.6) (end 131 82.5) (width 0.2) (layer "F.Cu") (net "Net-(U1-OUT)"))
 (segment (start 124 91.7) (end 124 92.674999) (width 0.2) (layer "F.Cu") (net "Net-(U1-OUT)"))
 (segment (start 131.1 92.330635) (end 131.1 82.6) (width 0.2) (layer "F.Cu") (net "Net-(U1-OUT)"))
 (segment (start 124.300001 92.975) (end 130.455635 92.975) (width 0.2) (layer "F.Cu") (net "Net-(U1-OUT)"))
 (segment (start 124 92.674999) (end 124.300001 92.975) (width 0.2) (layer "F.Cu") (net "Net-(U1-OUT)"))
 (segment (start 130.455635 92.975) (end 131.1 92.330635) (width 0.2) (layer "F.Cu") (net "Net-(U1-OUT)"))
 (segment (start 129.5 82.5) (end 128.845 83.155) (width 0.2) (layer "B.Cu") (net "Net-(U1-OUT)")))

